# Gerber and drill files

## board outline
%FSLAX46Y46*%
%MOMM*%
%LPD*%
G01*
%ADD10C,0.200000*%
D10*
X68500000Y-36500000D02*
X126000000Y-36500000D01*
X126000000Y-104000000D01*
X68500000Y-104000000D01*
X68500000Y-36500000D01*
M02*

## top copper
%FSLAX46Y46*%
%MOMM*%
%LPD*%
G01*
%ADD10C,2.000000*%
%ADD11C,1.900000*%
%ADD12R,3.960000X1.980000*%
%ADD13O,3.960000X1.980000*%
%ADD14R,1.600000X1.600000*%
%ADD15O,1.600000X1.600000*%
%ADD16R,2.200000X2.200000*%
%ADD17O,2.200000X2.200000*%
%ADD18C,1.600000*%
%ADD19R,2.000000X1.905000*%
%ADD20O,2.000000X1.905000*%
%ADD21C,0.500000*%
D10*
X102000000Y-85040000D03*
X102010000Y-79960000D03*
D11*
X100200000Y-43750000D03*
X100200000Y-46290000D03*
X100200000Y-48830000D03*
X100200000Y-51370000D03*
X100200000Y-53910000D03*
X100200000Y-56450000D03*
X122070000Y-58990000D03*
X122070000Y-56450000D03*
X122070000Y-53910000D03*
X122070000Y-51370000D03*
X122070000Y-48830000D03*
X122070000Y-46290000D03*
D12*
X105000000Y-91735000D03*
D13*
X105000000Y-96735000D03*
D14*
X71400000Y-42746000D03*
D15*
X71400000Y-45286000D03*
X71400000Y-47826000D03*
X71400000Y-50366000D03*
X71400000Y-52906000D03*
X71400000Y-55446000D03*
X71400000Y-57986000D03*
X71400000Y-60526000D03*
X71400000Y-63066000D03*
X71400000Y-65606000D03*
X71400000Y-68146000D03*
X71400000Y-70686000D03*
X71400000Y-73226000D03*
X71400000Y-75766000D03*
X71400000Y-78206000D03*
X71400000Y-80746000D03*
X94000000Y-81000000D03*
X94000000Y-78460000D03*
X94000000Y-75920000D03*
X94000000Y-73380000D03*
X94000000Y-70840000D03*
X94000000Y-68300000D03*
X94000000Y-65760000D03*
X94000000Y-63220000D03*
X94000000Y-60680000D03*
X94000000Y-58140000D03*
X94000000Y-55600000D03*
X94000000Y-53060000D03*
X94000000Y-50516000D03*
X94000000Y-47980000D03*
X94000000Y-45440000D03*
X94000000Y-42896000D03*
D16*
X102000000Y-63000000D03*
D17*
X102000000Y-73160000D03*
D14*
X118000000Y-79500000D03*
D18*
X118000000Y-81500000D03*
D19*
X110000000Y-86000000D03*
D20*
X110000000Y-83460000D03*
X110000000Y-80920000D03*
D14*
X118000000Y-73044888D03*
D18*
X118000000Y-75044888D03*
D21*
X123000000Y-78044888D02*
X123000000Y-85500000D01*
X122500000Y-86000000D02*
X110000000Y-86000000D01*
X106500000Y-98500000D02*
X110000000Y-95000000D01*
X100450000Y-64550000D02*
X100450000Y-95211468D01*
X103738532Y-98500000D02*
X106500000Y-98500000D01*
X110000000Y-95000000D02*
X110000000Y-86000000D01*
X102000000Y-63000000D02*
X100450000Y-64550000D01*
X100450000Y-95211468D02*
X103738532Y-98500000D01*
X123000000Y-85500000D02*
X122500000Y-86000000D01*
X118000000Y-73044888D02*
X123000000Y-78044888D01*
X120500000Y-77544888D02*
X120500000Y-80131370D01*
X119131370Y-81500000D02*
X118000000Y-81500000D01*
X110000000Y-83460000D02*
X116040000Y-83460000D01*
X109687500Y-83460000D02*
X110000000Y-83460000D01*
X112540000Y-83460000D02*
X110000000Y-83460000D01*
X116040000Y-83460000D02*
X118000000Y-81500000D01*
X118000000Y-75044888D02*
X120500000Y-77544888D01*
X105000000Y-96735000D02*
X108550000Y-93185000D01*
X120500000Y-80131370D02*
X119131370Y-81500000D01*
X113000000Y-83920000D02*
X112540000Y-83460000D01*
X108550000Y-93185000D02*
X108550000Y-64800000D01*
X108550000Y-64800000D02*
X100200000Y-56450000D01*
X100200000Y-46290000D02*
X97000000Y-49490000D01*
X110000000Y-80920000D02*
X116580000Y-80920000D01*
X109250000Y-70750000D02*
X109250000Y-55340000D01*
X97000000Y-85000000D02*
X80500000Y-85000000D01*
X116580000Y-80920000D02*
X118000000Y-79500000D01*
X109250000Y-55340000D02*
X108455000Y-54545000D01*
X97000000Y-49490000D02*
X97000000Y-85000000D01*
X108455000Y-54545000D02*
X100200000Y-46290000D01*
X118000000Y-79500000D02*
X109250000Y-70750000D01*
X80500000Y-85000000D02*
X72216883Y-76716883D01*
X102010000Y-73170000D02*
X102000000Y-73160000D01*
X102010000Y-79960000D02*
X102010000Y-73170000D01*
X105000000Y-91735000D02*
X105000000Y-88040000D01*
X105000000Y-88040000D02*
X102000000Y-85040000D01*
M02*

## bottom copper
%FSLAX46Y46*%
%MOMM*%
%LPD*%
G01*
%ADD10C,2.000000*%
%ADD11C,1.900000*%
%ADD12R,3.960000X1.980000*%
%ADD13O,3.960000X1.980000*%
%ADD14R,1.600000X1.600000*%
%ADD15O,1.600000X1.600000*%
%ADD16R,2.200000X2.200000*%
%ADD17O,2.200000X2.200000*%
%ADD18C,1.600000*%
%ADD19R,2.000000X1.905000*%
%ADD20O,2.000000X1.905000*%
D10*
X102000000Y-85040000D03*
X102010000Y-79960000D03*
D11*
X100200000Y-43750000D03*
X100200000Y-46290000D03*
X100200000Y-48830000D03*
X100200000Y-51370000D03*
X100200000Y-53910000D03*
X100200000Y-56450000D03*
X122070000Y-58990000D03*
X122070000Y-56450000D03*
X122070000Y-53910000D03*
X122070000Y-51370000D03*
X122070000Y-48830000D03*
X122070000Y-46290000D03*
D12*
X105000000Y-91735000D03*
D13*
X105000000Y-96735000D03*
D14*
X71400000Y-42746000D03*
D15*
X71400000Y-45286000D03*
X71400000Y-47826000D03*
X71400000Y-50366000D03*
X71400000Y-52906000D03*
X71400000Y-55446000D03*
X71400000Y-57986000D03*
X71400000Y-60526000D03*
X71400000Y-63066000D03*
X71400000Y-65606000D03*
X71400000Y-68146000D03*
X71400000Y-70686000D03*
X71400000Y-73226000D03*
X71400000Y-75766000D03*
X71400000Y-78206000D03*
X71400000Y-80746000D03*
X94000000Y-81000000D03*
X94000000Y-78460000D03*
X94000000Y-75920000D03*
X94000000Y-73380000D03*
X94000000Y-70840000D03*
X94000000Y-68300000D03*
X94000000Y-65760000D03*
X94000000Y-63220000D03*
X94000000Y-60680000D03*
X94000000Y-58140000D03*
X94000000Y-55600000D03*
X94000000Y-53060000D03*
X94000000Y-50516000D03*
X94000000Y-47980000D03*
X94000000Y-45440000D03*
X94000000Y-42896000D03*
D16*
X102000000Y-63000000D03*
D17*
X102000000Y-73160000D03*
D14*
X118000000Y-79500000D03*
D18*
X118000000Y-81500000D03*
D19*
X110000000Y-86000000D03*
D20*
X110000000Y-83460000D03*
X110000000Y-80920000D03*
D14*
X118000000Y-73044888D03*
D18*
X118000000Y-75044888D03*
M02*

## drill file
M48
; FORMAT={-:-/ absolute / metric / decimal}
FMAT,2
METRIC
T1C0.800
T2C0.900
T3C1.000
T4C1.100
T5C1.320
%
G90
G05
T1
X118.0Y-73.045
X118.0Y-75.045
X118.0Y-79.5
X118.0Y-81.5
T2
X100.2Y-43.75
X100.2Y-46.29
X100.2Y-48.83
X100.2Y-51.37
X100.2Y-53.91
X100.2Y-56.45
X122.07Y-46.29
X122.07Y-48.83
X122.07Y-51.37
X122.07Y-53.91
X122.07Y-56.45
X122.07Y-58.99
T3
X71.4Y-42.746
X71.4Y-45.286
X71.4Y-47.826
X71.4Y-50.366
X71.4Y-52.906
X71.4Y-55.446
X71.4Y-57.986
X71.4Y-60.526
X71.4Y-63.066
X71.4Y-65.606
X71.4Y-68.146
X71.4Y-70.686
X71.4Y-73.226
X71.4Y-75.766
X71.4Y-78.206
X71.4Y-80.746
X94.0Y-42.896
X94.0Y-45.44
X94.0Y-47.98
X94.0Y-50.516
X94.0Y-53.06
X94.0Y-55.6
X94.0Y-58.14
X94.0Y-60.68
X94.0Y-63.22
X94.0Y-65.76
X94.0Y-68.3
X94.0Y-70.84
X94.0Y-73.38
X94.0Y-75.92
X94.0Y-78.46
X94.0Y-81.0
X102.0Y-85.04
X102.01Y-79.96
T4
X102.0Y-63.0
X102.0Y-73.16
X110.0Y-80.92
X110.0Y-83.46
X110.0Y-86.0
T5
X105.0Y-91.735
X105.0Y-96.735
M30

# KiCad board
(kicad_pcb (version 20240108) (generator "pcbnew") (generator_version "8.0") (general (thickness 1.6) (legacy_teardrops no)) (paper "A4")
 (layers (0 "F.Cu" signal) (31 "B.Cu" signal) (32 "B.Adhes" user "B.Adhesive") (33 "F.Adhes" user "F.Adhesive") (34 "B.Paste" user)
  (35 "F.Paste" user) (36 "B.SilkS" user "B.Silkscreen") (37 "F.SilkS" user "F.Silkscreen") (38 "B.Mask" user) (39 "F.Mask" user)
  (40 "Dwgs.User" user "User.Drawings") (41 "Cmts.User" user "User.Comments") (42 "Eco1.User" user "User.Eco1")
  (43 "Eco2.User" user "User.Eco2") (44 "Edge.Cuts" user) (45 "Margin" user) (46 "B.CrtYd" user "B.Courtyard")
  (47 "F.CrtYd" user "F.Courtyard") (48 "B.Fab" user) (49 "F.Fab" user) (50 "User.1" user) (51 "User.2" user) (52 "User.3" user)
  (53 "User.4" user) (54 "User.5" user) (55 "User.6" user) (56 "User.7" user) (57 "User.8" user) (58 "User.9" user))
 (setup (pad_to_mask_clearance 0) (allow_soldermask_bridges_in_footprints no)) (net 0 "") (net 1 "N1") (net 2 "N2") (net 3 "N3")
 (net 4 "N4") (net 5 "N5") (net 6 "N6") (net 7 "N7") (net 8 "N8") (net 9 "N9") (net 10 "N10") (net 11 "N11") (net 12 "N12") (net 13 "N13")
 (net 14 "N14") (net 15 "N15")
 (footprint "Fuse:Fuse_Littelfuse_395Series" (layer "F.Cu") (at 102 85.04 90)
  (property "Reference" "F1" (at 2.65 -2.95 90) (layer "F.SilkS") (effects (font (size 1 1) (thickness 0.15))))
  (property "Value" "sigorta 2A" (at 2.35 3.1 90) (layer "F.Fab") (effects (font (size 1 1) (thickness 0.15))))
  (pad "1" thru_hole circle (at 0 0 90) (size 2 2) (drill 1) (layers "*.Cu" "*.Mask") (remove_unused_layers no) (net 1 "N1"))
  (pad "2" thru_hole circle (at 5.08 0.01 90) (size 2 2) (drill 1) (layers "*.Cu" "*.Mask") (remove_unused_layers no) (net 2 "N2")))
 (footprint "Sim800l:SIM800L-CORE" (layer "F.Cu") (at 100.2 43.75)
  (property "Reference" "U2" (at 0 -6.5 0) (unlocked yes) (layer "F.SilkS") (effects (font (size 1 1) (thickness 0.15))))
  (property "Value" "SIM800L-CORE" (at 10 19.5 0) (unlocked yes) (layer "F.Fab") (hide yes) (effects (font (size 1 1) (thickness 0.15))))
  (pad "1" thru_hole circle (at 0 0) (size 1.9 1.9) (drill 0.9) (layers "*.Cu" "*.Mask") (remove_unused_layers no) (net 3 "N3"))
  (pad "2" thru_hole circle (at 0 2.54) (size 1.9 1.9) (drill 0.9) (layers "*.Cu" "*.Mask") (remove_unused_layers no) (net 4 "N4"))
  (pad "3" thru_hole circle (at 0 5.08) (size 1.9 1.9) (drill 0.9) (layers "*.Cu" "*.Mask") (remove_unused_layers no) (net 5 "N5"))
  (pad "4" thru_hole circle (at 0 7.62) (size 1.9 1.9) (drill 0.9) (layers "*.Cu" "*.Mask") (remove_unused_layers no) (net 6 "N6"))
  (pad "5" thru_hole circle (at 0 10.16) (size 1.9 1.9) (drill 0.9) (layers "*.Cu" "*.Mask") (remove_unused_layers no) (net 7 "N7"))
  (pad "6" thru_hole circle (at 0 12.7) (size 1.9 1.9) (drill 0.9) (layers "*.Cu" "*.Mask") (remove_unused_layers no) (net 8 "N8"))
  (pad "7" thru_hole circle (at 21.87 15.24) (size 1.9 1.9) (drill 0.9) (layers "*.Cu" "*.Mask") (remove_unused_layers no) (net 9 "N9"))
  (pad "8" thru_hole circle (at 21.87 12.7) (size 1.9 1.9) (drill 0.9) (layers "*.Cu" "*.Mask") (remove_unused_layers no) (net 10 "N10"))
  (pad "9" thru_hole circle (at 21.87 10.16) (size 1.9 1.9) (drill 0.9) (layers "*.Cu" "*.Mask") (remove_unused_layers no) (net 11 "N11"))
  (pad "10" thru_hole circle (at 21.87 7.62) (size 1.9 1.9) (drill 0.9) (layers "*.Cu" "*.Mask") (remove_unused_layers no) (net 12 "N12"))
  (pad "11" thru_hole circle (at 21.87 5.08) (size 1.9 1.9) (drill 0.9) (layers "*.Cu" "*.Mask") (remove_unused_layers no) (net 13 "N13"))
  (pad "12" thru_hole circle (at 21.87 2.54) (size 1.9 1.9) (drill 0.9) (layers "*.Cu" "*.Mask") (remove_unused_layers no) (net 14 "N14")))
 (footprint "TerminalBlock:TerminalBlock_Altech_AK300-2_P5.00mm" (layer "F.Cu") (at 105 91.735 -90)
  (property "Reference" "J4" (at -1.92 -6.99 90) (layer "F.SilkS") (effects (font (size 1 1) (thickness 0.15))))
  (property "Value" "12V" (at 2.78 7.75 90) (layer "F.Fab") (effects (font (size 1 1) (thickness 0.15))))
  (pad "1" thru_hole rect (at 0 0 270) (size 1.98 3.96) (drill 1.32) (layers "*.Cu" "*.Mask") (remove_unused_layers no) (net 1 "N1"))
  (pad "2" thru_hole oval (at 5 0 270) (size 1.98 3.96) (drill 1.32) (layers "*.Cu" "*.Mask") (remove_unused_layers no) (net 8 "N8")))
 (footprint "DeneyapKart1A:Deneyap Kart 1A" (layer "F.Cu") (at 71.4 42.746)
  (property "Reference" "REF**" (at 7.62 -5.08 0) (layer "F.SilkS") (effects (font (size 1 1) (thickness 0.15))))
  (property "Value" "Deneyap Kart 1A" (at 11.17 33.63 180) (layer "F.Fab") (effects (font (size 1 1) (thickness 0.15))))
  (pad "1" thru_hole rect (at 0 0) (size 1.6 1.6) (drill 1) (layers "*.Cu" "*.Mask") (remove_unused_layers no))
  (pad "2" thru_hole oval (at 0 2.54) (size 1.6 1.6) (drill 1) (layers "*.Cu" "*.Mask") (remove_unused_layers no))
  (pad "3" thru_hole oval (at 0 5.08) (size 1.6 1.6) (drill 1) (layers "*.Cu" "*.Mask") (remove_unused_layers no))
  (pad "4" thru_hole oval (at 0 7.62) (size 1.6 1.6) (drill 1) (layers "*.Cu" "*.Mask") (remove_unused_layers no))
  (pad "5" thru_hole oval (at 0 10.16) (size 1.6 1.6) (drill 1) (layers "*.Cu" "*.Mask") (remove_unused_layers no))
  (pad "6" thru_hole oval (at 0 12.7) (size 1.6 1.6) (drill 1) (layers "*.Cu" "*.Mask") (remove_unused_layers no))
  (pad "7" thru_hole oval (at 0 15.24) (size 1.6 1.6) (drill 1) (layers "*.Cu" "*.Mask") (remove_unused_layers no))
  (pad "8" thru_hole oval (at 0 17.78) (size 1.6 1.6) (drill 1) (layers "*.Cu" "*.Mask") (remove_unused_layers no))
  (pad "9" thru_hole oval (at 0 20.32) (size 1.6 1.6) (drill 1) (layers "*.Cu" "*.Mask") (remove_unused_layers no))
  (pad "10" thru_hole oval (at 0 22.86) (size 1.6 1.6) (drill 1) (layers "*.Cu" "*.Mask") (remove_unused_layers no))
  (pad "11" thru_hole oval (at 0 25.4) (size 1.6 1.6) (drill 1) (layers "*.Cu" "*.Mask") (remove_unused_layers no))
  (pad "12" thru_hole oval (at 0 27.94) (size 1.6 1.6) (drill 1) (layers "*.Cu" "*.Mask") (remove_unused_layers no))
  (pad "13" thru_hole oval (at 0 30.48) (size 1.6 1.6) (drill 1) (layers "*.Cu" "*.Mask") (remove_unused_layers no))
  (pad "14" thru_hole oval (at 0 33.02) (size 1.6 1.6) (drill 1) (layers "*.Cu" "*.Mask") (remove_unused_layers no))
  (pad "15" thru_hole oval (at 0 35.46) (size 1.6 1.6) (drill 1) (layers "*.Cu" "*.Mask") (remove_unused_layers no))
  (pad "16" thru_hole oval (at 0 38) (size 1.6 1.6) (drill 1) (layers "*.Cu" "*.Mask") (remove_unused_layers no))
  (pad "17" thru_hole oval (at 22.6 38.254) (size 1.6 1.6) (drill 1) (layers "*.Cu" "*.Mask") (remove_unused_layers no))
  (pad "18" thru_hole oval (at 22.6 35.714) (size 1.6 1.6) (drill 1) (layers "*.Cu" "*.Mask") (remove_unused_layers no))
  (pad "19" thru_hole oval (at 22.6 33.174) (size 1.6 1.6) (drill 1) (layers "*.Cu" "*.Mask") (remove_unused_layers no))
  (pad "20" thru_hole oval (at 22.6 30.634) (size 1.6 1.6) (drill 1) (layers "*.Cu" "*.Mask") (remove_unused_layers no))
  (pad "21" thru_hole oval (at 22.6 28.094) (size 1.6 1.6) (drill 1) (layers "*.Cu" "*.Mask") (remove_unused_layers no))
  (pad "22" thru_hole oval (at 22.6 25.554) (size 1.6 1.6) (drill 1) (layers "*.Cu" "*.Mask") (remove_unused_layers no))
  (pad "23" thru_hole oval (at 22.6 23.014) (size 1.6 1.6) (drill 1) (layers "*.Cu" "*.Mask") (remove_unused_layers no))
  (pad "24" thru_hole oval (at 22.6 20.474) (size 1.6 1.6) (drill 1) (layers "*.Cu" "*.Mask") (remove_unused_layers no))
  (pad "25" thru_hole oval (at 22.6 17.934) (size 1.6 1.6) (drill 1) (layers "*.Cu" "*.Mask") (remove_unused_layers no))
  (pad "26" thru_hole oval (at 22.6 15.394) (size 1.6 1.6) (drill 1) (layers "*.Cu" "*.Mask") (remove_unused_layers no))
  (pad "27" thru_hole oval (at 22.6 12.854) (size 1.6 1.6) (drill 1) (layers "*.Cu" "*.Mask") (remove_unused_layers no))
  (pad "28" thru_hole oval (at 22.6 10.314) (size 1.6 1.6) (drill 1) (layers "*.Cu" "*.Mask") (remove_unused_layers no))
  (pad "29" thru_hole oval (at 22.6 7.77) (size 1.6 1.6) (drill 1) (layers "*.Cu" "*.Mask") (remove_unused_layers no))
  (pad "30" thru_hole oval (at 22.6 5.234) (size 1.6 1.6) (drill 1) (layers "*.Cu" "*.Mask") (remove_unused_layers no))
  (pad "31" thru_hole oval (at 22.6 2.694) (size 1.6 1.6) (drill 1) (layers "*.Cu" "*.Mask") (remove_unused_layers no))
  (pad "32" thru_hole oval (at 22.6 0.15) (size 1.6 1.6) (drill 1) (layers "*.Cu" "*.Mask") (remove_unused_layers no)))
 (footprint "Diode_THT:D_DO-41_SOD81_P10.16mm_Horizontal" (layer "F.Cu") (at 102 63 -90)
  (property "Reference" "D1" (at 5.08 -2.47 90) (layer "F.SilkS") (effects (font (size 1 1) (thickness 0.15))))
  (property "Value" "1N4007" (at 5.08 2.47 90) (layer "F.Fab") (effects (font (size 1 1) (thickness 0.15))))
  (pad "1" thru_hole rect (at 0 0 270) (size 2.2 2.2) (drill 1.1) (layers "*.Cu" "*.Mask") (remove_unused_layers no) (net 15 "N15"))
  (pad "2" thru_hole oval (at 10.16 0 270) (size 2.2 2.2) (drill 1.1) (layers "*.Cu" "*.Mask") (remove_unused_layers no) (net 2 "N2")))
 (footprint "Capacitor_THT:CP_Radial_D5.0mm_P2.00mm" (layer "F.Cu") (at 118 79.5 -90)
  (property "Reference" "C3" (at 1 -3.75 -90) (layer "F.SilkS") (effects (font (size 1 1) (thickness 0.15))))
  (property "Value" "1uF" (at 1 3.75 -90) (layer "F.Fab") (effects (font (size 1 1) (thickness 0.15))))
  (pad "1" thru_hole rect (at 0 0 270) (size 1.6 1.6) (drill 0.8) (layers "*.Cu" "*.Mask") (remove_unused_layers no) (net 4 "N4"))
  (pad "2" thru_hole circle (at 2 0 270) (size 1.6 1.6) (drill 0.8) (layers "*.Cu" "*.Mask") (remove_unused_layers no) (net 8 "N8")))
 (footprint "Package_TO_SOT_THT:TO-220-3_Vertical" (layer "F.Cu") (at 110 86 90)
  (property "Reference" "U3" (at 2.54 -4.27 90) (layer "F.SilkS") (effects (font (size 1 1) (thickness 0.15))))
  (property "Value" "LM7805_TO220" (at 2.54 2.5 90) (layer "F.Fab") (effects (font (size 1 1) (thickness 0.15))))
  (pad "1" thru_hole rect (at 0 0 90) (size 1.905 2) (drill 1.1) (layers "*.Cu" "*.Mask") (remove_unused_layers no) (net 15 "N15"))
  (pad "2" thru_hole oval (at 2.54 0 90) (size 1.905 2) (drill 1.1) (layers "*.Cu" "*.Mask") (remove_unused_layers no) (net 8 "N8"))
  (pad "3" thru_hole oval (at 5.08 0 90) (size 1.905 2) (drill 1.1) (layers "*.Cu" "*.Mask") (remove_unused_layers no) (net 4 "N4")))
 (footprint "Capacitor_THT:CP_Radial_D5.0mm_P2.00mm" (layer "F.Cu") (at 118 73.044888 -90)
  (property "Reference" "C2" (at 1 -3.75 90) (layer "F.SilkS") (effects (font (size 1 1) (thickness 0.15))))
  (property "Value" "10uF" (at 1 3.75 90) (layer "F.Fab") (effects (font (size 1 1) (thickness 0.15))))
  (pad "1" thru_hole rect (at 0 0 270) (size 1.6 1.6) (drill 0.8) (layers "*.Cu" "*.Mask") (remove_unused_layers no) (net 15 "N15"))
  (pad "2" thru_hole circle (at 2 0 270) (size 1.6 1.6) (drill 0.8) (layers "*.Cu" "*.Mask") (remove_unused_layers no) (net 8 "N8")))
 (gr_rect (start 68.5 36.5) (end 126 104) (stroke (width 0.2) (type default)) (fill none) (layer "Edge.Cuts"))
 (segment (start 123 78.044888) (end 123 85.5) (width 0.5) (layer "F.Cu") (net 15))
 (segment (start 122.5 86) (end 110 86) (width 0.5) (layer "F.Cu") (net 15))
 (segment (start 106.5 98.5) (end 110 95) (width 0.5) (layer "F.Cu") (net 15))
 (segment (start 100.45 64.55) (end 100.45 95.211468) (width 0.5) (layer "F.Cu") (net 15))
 (segment (start 103.738532 98.5) (end 106.5 98.5) (width 0.5) (layer "F.Cu") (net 15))
 (segment (start 110 95) (end 110 86) (width 0.5) (layer "F.Cu") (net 15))
 (segment (start 102 63) (end 100.45 64.55) (width 0.5) (layer "F.Cu") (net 15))
 (segment (start 100.45 95.211468) (end 103.738532 98.5) (width 0.5) (layer "F.Cu") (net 15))
 (segment (start 123 85.5) (end 122.5 86) (width 0.5) (layer "F.Cu") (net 15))
 (segment (start 118 73.044888) (end 123 78.044888) (width 0.5) (layer "F.Cu") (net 15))
 (segment (start 120.5 77.544888) (end 120.5 80.13137) (width 0.5) (layer "F.Cu") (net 8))
 (segment (start 119.13137 81.5) (end 118 81.5) (width 0.5) (layer "F.Cu") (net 8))
 (segment (start 110 83.46) (end 116.04 83.46) (width 0.5) (layer "F.Cu") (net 8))
 (segment (start 109.6875 83.46) (end 110 83.46) (width 0.5) (layer "F.Cu") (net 8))
 (segment (start 112.54 83.46) (end 110 83.46) (width 0.5) (layer "F.Cu") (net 8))
 (segment (start 116.04 83.46) (end 118 81.5) (width 0.5) (layer "F.Cu") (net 8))
 (segment (start 118 75.044888) (end 120.5 77.544888) (width 0.5) (layer "F.Cu") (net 8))
 (segment (start 105 96.735) (end 108.55 93.185) (width 0.5) (layer "F.Cu") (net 8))
 (segment (start 120.5 80.13137) (end 119.13137 81.5) (width 0.5) (layer "F.Cu") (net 8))
 (segment (start 113 83.92) (end 112.54 83.46) (width 0.5) (layer "F.Cu") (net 8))
 (segment (start 108.55 93.185) (end 108.55 64.8) (width 0.5) (layer "F.Cu") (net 8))
 (segment (start 108.55 64.8) (end 100.2 56.45) (width 0.5) (layer "F.Cu") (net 8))
 (segment (start 100.2 46.29) (end 97 49.49) (width 0.5) (layer "F.Cu") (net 4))
 (segment (start 110 80.92) (end 116.58 80.92) (width 0.5) (layer "F.Cu") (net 4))
 (segment (start 109.25 70.75) (end 109.25 55.34) (width 0.5) (layer "F.Cu") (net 4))
 (segment (start 97 85) (end 80.5 85) (width 0.5) (layer "F.Cu") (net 4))
 (segment (start 116.58 80.92) (end 118 79.5) (width 0.5) (layer "F.Cu") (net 4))
 (segment (start 109.25 55.34) (end 108.455 54.545) (width 0.5) (layer "F.Cu") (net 4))
 (segment (start 97 49.49) (end 97 85) (width 0.5) (layer "F.Cu") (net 4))
 (segment (start 108.455 54.545) (end 100.2 46.29) (width 0.5) (layer "F.Cu") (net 4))
 (segment (start 118 79.5) (end 109.25 70.75) (width 0.5) (layer "F.Cu") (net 4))
 (segment (start 80.5 85) (end 72.216883 76.716883) (width 0.5) (layer "F.Cu") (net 4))
 (segment (start 102.01 73.17) (end 102 73.16) (width 0.5) (layer "F.Cu") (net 2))
 (segment (start 102.01 79.96) (end 102.01 73.17) (width 0.5) (layer "F.Cu") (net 2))
 (segment (start 105 91.735) (end 105 88.04) (width 0.5) (layer "F.Cu") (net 1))
 (segment (start 105 88.04) (end 102 85.04) (width 0.5) (layer "F.Cu") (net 1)))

